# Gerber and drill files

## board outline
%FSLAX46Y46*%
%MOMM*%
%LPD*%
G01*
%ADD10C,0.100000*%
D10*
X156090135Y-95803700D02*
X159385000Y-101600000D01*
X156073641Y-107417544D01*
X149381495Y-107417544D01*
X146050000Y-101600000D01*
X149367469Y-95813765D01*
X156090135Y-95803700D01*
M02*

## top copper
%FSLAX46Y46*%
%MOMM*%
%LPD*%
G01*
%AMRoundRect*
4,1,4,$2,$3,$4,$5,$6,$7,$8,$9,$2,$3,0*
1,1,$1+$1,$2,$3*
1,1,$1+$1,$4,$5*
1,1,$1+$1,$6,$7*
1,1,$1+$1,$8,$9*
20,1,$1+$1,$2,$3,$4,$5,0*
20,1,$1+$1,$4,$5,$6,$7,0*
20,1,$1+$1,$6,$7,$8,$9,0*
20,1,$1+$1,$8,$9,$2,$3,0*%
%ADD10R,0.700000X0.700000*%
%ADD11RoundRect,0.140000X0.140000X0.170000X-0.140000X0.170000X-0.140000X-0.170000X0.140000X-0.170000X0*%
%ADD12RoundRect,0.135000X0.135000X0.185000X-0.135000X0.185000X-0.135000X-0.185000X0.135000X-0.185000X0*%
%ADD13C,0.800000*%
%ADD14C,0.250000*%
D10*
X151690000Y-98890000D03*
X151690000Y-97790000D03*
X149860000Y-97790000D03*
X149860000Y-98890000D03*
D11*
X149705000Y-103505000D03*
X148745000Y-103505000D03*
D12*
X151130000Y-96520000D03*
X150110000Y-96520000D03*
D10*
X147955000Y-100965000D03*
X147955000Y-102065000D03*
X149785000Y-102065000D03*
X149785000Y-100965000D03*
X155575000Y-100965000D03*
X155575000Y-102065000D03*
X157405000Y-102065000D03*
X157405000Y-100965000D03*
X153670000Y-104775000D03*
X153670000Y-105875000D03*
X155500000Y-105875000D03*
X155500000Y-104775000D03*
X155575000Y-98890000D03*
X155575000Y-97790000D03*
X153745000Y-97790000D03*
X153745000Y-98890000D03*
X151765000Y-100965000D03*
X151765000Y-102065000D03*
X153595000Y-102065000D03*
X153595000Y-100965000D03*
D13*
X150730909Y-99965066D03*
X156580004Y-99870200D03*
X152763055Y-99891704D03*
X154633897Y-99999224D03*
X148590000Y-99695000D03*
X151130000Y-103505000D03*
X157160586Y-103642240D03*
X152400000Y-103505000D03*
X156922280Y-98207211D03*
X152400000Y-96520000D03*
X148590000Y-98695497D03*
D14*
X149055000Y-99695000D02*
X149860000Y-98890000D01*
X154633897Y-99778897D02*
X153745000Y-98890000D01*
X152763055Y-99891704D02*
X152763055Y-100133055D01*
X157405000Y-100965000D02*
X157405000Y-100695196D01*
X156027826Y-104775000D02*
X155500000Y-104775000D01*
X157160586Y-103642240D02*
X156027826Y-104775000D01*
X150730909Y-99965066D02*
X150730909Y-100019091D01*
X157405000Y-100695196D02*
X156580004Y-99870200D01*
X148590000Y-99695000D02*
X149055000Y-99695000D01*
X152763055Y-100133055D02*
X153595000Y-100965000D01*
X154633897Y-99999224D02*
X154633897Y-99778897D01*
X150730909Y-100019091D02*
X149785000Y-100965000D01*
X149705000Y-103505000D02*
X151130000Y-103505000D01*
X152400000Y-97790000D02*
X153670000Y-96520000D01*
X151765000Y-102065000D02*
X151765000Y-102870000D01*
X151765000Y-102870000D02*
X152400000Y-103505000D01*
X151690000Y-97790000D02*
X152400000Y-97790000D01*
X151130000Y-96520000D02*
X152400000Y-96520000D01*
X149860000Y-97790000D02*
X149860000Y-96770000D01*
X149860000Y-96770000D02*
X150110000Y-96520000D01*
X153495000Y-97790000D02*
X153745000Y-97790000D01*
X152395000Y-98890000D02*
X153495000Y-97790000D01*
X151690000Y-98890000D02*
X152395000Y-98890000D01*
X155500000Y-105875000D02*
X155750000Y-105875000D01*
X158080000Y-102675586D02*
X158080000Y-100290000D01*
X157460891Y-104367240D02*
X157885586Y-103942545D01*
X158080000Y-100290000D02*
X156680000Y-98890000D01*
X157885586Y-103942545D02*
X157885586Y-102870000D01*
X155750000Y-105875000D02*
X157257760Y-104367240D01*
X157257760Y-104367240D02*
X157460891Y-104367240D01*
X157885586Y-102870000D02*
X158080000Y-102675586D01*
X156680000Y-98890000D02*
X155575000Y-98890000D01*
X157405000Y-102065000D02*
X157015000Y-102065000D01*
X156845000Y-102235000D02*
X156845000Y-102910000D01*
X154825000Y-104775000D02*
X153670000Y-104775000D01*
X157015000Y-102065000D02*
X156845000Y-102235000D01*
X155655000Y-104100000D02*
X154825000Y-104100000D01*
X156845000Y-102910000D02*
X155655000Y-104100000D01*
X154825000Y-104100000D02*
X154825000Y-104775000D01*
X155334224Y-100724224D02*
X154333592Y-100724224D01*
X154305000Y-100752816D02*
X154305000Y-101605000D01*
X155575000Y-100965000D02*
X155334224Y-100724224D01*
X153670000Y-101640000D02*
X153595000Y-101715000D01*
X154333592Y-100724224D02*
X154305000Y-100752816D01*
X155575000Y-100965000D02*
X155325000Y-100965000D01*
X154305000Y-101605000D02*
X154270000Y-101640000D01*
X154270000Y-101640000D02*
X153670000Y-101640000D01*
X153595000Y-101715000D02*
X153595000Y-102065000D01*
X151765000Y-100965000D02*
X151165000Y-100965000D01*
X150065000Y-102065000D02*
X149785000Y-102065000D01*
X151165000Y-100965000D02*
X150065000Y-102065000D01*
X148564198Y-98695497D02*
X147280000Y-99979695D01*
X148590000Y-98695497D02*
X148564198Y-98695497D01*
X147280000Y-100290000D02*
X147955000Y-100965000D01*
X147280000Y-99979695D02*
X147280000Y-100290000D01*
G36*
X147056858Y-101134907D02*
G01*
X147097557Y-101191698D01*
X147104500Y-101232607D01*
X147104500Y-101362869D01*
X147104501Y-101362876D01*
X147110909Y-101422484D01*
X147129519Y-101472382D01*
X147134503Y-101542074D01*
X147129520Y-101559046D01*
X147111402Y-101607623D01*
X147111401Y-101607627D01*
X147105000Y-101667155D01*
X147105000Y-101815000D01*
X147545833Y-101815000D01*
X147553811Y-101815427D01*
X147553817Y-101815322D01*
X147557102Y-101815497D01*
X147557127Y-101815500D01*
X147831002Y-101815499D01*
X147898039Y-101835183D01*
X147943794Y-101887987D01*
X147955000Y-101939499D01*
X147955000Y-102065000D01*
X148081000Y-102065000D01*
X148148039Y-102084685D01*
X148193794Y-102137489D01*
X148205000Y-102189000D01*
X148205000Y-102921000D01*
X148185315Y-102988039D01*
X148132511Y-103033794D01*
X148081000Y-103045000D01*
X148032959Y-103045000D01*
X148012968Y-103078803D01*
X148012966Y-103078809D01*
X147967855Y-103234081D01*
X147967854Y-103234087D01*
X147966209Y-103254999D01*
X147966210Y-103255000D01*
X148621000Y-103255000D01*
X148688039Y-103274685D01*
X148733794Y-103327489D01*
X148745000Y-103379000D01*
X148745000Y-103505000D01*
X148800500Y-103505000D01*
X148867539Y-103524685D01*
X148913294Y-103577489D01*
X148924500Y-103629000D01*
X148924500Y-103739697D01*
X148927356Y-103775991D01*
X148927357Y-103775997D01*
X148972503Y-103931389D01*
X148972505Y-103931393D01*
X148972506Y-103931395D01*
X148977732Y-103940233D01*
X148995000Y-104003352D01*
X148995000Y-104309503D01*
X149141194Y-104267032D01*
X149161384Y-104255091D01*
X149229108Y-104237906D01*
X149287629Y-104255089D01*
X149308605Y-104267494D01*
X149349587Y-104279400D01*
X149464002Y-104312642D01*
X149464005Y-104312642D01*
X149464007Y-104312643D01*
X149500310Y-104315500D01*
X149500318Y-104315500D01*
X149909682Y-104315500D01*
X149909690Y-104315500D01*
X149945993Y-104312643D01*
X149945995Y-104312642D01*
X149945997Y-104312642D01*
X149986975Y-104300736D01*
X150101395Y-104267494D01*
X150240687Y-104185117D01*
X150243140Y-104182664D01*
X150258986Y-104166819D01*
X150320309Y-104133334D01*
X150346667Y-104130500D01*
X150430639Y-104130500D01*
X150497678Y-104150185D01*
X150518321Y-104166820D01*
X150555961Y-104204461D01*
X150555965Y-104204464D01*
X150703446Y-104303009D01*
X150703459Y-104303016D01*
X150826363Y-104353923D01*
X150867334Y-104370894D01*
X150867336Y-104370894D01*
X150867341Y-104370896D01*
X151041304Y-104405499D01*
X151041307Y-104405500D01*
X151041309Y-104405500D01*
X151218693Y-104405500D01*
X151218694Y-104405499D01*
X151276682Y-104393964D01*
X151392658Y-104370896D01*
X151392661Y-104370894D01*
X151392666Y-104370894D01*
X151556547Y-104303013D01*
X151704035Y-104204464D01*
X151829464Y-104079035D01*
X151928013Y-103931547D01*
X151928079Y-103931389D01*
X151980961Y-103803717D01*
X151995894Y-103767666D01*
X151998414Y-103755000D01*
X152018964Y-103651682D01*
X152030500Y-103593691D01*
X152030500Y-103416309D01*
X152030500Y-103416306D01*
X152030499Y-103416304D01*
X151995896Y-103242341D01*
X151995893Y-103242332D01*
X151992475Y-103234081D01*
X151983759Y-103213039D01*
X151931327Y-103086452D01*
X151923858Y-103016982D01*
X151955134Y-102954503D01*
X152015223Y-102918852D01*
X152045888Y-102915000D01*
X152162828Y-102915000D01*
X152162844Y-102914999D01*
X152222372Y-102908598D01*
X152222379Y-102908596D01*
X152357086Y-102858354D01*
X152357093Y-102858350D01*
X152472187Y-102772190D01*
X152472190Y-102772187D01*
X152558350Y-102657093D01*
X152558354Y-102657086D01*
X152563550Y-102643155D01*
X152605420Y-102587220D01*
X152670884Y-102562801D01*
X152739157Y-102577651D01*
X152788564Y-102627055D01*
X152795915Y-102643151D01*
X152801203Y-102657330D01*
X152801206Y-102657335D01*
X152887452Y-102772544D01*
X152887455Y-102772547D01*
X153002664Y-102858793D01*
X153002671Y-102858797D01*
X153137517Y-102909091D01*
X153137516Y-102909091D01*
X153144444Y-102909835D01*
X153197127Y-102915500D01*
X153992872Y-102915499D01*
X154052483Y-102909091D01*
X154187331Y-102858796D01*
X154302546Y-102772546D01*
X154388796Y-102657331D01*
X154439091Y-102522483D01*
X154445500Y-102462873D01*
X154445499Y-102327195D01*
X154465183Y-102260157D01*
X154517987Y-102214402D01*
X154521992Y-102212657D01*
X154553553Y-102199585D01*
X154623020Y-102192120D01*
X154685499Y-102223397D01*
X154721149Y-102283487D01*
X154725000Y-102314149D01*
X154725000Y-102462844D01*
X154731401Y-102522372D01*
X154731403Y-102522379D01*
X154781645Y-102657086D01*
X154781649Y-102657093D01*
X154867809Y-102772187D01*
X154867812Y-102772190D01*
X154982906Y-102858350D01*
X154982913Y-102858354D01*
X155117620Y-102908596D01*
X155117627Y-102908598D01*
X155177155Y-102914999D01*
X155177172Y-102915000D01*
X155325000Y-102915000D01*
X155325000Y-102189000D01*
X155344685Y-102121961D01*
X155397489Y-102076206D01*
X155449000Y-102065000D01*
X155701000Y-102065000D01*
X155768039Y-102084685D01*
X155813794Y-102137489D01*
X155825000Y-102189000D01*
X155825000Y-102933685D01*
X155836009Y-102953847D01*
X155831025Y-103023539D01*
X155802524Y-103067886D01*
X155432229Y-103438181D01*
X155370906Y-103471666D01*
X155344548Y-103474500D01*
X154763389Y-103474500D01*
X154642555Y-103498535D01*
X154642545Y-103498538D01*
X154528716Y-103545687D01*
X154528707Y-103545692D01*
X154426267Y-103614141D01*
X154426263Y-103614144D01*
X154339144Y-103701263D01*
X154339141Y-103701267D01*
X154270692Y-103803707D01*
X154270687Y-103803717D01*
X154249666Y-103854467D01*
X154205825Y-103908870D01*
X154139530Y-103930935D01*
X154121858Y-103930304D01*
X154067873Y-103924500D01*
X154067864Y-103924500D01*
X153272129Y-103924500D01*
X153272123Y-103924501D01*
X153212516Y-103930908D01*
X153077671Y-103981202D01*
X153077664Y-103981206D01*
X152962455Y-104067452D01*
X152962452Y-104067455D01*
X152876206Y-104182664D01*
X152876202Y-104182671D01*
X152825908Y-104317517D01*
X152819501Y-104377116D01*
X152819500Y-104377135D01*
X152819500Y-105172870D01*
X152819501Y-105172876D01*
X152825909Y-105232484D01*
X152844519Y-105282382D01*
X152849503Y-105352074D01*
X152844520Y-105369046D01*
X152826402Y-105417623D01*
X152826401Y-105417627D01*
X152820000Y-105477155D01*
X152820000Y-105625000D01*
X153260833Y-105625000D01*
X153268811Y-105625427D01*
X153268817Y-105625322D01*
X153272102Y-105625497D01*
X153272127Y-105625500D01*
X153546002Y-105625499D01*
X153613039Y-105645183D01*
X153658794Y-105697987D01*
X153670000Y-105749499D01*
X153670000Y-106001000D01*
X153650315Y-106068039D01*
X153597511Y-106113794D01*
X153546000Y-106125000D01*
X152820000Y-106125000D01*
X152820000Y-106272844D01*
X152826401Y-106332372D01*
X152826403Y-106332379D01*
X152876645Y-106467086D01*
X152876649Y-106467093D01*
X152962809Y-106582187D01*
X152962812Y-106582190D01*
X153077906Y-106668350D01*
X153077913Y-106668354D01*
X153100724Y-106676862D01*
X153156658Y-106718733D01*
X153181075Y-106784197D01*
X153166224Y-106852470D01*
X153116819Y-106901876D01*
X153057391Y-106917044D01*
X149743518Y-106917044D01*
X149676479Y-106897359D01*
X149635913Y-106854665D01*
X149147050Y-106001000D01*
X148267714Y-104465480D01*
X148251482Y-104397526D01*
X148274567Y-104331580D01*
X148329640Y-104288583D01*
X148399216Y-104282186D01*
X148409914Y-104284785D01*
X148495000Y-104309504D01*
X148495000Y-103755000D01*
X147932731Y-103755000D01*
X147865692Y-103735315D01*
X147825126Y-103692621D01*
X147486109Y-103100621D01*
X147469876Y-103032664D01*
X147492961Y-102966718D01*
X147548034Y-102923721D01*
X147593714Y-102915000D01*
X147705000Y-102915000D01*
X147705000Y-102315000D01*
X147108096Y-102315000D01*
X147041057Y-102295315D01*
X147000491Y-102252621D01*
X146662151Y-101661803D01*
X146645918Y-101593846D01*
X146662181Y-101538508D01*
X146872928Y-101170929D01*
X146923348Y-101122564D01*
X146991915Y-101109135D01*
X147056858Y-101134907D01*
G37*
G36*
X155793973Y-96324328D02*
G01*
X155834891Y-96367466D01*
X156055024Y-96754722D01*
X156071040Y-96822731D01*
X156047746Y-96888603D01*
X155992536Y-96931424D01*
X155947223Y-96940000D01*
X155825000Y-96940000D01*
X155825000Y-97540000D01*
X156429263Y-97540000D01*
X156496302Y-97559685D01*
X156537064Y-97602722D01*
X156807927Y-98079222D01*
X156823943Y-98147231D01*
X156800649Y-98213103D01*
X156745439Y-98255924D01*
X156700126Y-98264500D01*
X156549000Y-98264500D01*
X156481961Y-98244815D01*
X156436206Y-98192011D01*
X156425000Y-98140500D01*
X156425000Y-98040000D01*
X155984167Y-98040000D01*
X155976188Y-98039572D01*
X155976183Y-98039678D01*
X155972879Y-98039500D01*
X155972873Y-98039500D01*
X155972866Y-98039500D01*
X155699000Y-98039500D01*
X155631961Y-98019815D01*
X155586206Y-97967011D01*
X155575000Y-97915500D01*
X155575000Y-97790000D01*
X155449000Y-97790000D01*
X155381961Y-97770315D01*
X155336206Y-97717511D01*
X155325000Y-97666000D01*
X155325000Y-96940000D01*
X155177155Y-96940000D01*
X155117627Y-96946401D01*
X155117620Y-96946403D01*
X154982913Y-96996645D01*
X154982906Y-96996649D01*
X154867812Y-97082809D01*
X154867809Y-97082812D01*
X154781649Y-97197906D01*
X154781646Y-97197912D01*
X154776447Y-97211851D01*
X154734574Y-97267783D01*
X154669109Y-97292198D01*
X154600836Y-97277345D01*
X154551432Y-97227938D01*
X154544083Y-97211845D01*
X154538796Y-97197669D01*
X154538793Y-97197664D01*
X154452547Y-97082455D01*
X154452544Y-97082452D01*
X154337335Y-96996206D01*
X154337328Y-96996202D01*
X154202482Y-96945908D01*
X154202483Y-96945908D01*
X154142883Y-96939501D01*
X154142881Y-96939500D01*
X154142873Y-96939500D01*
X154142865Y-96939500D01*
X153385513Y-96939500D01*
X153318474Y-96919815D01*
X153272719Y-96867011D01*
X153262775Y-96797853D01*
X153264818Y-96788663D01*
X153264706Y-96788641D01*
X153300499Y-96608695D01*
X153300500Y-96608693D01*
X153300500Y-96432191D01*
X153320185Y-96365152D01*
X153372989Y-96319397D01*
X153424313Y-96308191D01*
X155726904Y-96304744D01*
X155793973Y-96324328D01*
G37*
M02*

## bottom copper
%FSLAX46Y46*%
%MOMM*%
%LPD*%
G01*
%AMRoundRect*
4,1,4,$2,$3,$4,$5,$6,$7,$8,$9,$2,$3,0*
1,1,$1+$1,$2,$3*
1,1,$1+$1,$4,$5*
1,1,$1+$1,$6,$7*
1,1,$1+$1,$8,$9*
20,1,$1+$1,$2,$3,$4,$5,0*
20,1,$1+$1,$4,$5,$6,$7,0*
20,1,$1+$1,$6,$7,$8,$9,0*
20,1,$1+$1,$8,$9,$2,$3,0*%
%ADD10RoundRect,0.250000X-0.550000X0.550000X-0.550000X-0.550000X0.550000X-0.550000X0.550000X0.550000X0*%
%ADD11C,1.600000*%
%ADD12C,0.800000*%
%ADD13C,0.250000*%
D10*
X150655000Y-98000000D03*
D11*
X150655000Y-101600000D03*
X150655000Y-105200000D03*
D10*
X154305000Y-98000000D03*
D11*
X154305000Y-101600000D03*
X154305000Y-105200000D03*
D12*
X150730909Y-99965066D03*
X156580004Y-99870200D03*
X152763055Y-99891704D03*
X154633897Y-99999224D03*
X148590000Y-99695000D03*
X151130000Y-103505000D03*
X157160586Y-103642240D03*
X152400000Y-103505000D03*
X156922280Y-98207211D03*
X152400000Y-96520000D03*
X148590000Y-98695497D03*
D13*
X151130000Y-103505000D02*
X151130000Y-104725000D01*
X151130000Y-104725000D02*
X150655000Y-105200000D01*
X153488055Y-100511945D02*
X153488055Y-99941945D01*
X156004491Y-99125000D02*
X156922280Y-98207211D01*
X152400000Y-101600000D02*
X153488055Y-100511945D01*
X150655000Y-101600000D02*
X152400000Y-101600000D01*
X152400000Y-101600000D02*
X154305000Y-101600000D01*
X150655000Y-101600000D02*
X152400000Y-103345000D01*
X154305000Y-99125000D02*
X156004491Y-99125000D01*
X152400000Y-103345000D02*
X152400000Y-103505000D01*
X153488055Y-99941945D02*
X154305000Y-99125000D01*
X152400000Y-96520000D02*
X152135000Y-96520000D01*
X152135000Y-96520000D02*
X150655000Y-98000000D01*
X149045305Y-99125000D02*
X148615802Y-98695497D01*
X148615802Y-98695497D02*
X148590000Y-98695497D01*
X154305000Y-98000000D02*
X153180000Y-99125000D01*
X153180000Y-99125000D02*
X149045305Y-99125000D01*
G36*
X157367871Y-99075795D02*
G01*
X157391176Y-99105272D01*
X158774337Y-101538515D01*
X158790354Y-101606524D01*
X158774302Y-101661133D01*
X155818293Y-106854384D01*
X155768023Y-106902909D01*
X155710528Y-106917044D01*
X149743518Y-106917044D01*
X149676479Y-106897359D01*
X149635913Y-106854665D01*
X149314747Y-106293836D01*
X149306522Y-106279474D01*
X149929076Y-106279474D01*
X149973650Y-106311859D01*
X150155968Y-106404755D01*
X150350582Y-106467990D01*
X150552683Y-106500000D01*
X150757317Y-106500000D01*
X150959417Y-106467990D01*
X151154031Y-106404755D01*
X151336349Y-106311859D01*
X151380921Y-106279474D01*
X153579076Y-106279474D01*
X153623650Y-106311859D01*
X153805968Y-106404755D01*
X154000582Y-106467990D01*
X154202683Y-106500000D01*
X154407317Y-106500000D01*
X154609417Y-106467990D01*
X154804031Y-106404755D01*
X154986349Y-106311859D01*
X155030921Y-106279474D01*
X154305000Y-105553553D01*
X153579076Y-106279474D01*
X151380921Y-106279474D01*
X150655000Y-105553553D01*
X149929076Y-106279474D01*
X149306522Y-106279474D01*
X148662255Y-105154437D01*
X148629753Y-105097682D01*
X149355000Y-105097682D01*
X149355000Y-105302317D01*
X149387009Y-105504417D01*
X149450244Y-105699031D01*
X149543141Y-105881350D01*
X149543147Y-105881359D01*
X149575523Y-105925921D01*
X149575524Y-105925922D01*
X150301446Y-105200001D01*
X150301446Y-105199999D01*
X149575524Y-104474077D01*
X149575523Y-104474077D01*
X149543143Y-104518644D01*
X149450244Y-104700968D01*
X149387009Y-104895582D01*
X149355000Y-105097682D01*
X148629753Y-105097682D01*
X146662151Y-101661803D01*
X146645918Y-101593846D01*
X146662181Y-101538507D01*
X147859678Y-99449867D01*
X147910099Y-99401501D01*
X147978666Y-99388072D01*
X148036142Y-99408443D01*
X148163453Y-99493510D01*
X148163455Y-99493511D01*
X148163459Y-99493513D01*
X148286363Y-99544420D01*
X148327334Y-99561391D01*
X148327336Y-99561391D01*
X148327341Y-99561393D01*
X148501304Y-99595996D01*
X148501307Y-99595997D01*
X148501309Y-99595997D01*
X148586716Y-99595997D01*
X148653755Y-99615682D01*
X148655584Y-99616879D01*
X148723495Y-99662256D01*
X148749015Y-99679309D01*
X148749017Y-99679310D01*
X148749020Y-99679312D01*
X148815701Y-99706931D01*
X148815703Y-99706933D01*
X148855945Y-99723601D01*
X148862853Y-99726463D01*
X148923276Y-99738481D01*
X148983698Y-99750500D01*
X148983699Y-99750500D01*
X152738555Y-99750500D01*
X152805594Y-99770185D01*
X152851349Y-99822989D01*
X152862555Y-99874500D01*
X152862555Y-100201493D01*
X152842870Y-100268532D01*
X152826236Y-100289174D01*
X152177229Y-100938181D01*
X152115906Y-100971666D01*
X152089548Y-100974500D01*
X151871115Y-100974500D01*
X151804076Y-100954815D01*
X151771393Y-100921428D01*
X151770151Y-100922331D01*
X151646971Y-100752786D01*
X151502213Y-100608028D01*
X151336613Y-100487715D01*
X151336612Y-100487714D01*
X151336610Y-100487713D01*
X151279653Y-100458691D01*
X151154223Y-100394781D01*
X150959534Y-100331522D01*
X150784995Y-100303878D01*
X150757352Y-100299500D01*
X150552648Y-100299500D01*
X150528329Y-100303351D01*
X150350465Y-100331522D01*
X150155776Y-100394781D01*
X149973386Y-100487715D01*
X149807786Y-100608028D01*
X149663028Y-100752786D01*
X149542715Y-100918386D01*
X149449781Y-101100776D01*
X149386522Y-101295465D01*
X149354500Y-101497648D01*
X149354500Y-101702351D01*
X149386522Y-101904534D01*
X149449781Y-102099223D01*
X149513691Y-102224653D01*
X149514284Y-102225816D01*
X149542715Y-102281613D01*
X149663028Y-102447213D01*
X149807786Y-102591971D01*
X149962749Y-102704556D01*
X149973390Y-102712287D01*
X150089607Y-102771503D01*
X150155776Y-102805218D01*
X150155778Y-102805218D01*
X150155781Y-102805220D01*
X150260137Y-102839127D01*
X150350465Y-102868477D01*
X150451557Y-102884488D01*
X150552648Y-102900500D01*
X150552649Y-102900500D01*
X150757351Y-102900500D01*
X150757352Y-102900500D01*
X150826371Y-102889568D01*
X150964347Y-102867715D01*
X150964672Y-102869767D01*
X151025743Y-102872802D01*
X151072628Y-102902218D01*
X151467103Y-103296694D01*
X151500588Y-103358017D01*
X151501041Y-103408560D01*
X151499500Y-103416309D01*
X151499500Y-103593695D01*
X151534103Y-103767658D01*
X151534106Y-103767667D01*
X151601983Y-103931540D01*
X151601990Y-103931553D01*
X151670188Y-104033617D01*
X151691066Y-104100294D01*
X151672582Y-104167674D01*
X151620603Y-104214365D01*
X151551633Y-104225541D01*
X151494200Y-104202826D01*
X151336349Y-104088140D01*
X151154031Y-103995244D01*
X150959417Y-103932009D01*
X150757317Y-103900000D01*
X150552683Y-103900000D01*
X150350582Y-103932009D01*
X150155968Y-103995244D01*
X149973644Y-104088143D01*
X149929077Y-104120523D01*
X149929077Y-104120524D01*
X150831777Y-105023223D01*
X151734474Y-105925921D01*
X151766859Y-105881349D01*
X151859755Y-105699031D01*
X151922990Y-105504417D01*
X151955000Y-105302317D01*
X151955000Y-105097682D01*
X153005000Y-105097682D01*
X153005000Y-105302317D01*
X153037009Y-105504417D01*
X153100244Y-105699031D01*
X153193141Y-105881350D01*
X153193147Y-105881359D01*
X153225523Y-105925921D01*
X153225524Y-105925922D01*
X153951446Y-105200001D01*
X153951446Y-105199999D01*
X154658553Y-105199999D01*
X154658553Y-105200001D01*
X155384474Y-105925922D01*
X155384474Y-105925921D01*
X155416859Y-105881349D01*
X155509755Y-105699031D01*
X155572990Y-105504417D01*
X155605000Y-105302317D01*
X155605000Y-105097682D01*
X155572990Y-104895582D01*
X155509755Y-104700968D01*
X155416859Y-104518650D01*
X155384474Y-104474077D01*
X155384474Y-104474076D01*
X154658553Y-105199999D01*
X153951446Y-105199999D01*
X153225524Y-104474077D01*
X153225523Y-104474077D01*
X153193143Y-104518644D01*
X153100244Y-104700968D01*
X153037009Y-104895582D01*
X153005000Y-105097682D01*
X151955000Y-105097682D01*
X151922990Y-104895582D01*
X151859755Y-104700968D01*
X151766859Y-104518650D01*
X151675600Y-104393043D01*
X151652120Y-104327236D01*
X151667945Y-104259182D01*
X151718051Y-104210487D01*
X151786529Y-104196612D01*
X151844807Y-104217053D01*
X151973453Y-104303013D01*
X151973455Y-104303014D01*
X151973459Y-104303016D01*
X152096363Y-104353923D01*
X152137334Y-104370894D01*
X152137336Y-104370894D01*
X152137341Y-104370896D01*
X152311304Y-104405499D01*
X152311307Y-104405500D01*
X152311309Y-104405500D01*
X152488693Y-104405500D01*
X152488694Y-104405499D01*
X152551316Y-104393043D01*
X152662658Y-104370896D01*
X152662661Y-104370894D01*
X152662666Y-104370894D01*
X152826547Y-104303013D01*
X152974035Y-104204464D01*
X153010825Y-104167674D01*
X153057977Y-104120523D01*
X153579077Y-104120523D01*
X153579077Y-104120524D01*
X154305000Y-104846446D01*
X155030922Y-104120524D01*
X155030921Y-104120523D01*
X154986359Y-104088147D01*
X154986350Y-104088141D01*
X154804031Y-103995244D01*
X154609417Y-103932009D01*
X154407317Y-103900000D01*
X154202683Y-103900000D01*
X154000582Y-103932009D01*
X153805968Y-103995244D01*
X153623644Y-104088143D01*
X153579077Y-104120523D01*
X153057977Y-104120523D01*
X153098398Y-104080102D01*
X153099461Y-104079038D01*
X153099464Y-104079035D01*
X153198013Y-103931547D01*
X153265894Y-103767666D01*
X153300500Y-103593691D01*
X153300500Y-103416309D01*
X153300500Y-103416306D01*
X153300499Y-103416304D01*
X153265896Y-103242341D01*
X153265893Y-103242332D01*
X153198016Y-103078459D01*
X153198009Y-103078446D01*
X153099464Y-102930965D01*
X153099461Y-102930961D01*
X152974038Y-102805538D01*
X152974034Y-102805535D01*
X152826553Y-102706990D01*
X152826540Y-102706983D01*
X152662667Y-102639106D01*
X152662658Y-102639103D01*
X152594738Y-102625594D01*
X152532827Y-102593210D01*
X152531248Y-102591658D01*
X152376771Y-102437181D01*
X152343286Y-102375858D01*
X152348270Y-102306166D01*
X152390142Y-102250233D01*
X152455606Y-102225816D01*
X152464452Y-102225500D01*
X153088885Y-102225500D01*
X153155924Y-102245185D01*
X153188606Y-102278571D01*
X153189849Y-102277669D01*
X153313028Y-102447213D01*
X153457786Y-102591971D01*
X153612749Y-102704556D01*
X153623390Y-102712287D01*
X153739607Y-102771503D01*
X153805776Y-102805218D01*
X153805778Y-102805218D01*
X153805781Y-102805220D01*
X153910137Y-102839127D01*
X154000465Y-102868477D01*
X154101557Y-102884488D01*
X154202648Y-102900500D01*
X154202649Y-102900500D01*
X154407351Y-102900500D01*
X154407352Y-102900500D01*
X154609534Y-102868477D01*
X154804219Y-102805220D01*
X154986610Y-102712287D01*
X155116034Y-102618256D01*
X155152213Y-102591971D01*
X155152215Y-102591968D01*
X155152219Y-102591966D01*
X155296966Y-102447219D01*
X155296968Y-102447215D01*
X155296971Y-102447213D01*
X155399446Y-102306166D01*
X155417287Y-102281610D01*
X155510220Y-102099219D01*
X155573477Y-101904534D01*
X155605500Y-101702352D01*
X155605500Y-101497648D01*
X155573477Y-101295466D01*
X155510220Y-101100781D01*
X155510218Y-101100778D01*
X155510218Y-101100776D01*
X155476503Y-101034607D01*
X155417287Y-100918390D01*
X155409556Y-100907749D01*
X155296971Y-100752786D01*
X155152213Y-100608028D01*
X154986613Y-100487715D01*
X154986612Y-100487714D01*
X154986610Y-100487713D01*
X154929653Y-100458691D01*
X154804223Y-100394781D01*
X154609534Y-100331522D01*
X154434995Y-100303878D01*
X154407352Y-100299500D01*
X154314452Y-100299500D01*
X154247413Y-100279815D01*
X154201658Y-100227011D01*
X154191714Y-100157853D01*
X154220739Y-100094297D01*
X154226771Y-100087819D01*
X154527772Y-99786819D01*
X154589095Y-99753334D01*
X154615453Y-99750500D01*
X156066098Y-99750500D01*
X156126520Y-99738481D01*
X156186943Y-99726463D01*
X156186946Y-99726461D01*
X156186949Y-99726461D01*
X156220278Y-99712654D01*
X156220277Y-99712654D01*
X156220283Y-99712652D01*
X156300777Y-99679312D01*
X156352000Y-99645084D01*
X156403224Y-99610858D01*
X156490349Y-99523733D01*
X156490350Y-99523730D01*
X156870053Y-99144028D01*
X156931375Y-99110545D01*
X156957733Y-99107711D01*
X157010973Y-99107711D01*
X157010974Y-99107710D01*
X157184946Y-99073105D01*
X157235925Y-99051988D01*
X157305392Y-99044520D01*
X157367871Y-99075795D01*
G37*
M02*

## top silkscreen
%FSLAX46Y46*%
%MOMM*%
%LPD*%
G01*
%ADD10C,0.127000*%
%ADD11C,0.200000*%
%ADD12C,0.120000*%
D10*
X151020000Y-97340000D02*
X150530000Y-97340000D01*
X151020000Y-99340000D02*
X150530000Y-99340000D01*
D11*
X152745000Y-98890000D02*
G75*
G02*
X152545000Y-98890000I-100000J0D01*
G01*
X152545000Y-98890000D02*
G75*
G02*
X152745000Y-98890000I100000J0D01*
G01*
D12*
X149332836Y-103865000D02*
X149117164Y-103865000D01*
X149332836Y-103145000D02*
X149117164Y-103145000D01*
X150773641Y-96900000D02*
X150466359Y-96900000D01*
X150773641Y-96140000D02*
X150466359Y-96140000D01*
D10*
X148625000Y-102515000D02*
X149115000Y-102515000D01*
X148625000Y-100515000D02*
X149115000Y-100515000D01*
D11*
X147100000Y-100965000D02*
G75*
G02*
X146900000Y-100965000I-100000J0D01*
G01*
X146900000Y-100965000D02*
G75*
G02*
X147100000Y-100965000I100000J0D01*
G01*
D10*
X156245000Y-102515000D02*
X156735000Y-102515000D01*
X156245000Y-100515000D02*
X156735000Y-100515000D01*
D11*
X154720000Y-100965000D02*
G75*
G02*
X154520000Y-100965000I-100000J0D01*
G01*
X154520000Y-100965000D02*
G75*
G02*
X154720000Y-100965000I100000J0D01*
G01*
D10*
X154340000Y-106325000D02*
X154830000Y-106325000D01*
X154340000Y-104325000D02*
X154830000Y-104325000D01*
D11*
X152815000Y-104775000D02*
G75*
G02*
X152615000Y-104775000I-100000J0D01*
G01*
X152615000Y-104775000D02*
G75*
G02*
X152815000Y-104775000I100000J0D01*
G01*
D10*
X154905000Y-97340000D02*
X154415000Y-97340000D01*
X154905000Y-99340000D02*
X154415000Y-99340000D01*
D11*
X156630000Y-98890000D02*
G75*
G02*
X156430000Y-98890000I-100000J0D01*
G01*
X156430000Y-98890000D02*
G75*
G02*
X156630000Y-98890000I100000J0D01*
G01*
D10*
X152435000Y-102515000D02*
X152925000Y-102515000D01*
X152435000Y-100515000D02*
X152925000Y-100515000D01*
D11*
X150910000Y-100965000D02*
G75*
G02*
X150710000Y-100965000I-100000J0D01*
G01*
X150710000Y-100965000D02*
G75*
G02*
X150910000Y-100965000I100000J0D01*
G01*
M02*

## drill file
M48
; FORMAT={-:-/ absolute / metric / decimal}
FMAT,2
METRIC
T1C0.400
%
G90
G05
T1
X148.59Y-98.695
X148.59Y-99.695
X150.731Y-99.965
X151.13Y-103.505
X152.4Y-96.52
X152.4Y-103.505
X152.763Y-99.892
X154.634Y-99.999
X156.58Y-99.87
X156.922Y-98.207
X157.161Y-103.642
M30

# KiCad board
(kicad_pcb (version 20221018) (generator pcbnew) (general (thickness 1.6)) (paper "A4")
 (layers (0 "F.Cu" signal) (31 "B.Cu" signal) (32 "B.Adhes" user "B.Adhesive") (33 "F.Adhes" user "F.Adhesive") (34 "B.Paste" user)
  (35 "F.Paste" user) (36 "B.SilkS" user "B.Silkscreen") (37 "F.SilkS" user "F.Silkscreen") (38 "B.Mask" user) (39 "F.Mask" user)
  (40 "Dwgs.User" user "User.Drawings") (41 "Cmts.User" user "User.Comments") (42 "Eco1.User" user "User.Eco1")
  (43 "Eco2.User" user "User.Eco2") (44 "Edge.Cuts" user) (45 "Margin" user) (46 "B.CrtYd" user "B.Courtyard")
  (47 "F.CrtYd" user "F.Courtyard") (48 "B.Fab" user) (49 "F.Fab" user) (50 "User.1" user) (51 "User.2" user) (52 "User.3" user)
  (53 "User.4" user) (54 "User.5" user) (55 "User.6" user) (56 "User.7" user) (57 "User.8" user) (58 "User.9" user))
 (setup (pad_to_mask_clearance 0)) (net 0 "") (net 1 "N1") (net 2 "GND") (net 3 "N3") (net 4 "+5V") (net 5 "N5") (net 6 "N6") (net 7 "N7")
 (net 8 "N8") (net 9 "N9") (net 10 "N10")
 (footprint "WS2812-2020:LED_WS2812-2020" (layer "F.Cu") (at 150.775 98.34)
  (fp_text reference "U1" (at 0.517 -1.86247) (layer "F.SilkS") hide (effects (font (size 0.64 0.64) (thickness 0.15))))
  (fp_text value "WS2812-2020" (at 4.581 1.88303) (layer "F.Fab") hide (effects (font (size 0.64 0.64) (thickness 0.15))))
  (fp_line (start 0.245 -1) (end -0.245 -1) (stroke (width 0.127) (type solid)) (layer "F.SilkS"))
  (fp_line (start 0.245 1) (end -0.245 1) (stroke (width 0.127) (type solid)) (layer "F.SilkS"))
  (fp_circle (center 1.87 0.55) (end 1.97 0.55) (stroke (width 0.2) (type solid)) (fill none) (layer "F.SilkS"))
  (pad "1" smd rect (at 0.915 0.55) (size 0.7 0.7) (layers "F.Cu" "F.Paste" "F.Mask") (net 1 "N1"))
  (pad "2" smd rect (at 0.915 -0.55) (size 0.7 0.7) (layers "F.Cu" "F.Paste" "F.Mask") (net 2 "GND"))
  (pad "3" smd rect (at -0.915 -0.55) (size 0.7 0.7) (layers "F.Cu" "F.Paste" "F.Mask") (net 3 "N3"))
  (pad "4" smd rect (at -0.915 0.55) (size 0.7 0.7) (layers "F.Cu" "F.Paste" "F.Mask") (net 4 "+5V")))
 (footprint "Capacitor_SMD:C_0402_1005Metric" (layer "F.Cu") (at 149.225 103.505 180)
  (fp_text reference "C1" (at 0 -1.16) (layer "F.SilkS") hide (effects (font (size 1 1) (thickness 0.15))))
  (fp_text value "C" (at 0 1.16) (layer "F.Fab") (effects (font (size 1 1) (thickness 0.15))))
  (fp_line (start -0.107836 -0.36) (end 0.107836 -0.36) (stroke (width 0.12) (type solid)) (layer "F.SilkS"))
  (fp_line (start -0.107836 0.36) (end 0.107836 0.36) (stroke (width 0.12) (type solid)) (layer "F.SilkS"))
  (pad "1" smd roundrect (at -0.48 0 180) (size 0.56 0.62) (layers "F.Cu" "F.Paste" "F.Mask") (roundrect_rratio 0.25) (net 4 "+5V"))
  (pad "2" smd roundrect (at 0.48 0 180) (size 0.56 0.62) (layers "F.Cu" "F.Paste" "F.Mask") (roundrect_rratio 0.25) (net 2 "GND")))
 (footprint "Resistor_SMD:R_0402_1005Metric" (layer "F.Cu") (at 150.62 96.52 180)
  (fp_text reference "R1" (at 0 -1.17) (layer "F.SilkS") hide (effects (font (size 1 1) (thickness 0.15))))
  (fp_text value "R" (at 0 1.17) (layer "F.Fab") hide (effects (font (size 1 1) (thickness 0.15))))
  (fp_line (start -0.153641 -0.38) (end 0.153641 -0.38) (stroke (width 0.12) (type solid)) (layer "F.SilkS"))
  (fp_line (start -0.153641 0.38) (end 0.153641 0.38) (stroke (width 0.12) (type solid)) (layer "F.SilkS"))
  (pad "1" smd roundrect (at -0.51 0 180) (size 0.54 0.64) (layers "F.Cu" "F.Paste" "F.Mask") (roundrect_rratio 0.25) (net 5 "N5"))
  (pad "2" smd roundrect (at 0.51 0 180) (size 0.54 0.64) (layers "F.Cu" "F.Paste" "F.Mask") (roundrect_rratio 0.25) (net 3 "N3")))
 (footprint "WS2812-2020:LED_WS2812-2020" (layer "F.Cu") (at 148.87 101.515 180)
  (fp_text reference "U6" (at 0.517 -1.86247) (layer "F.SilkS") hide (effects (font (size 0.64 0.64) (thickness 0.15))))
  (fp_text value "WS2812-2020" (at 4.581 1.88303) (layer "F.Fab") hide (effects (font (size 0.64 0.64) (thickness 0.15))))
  (fp_line (start 0.245 -1) (end -0.245 -1) (stroke (width 0.127) (type solid)) (layer "F.SilkS"))
  (fp_line (start 0.245 1) (end -0.245 1) (stroke (width 0.127) (type solid)) (layer "F.SilkS"))
  (fp_circle (center 1.87 0.55) (end 1.97 0.55) (stroke (width 0.2) (type solid)) (fill none) (layer "F.SilkS"))
  (pad "1" smd rect (at 0.915 0.55 180) (size 0.7 0.7) (layers "F.Cu" "F.Paste" "F.Mask") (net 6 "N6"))
  (pad "2" smd rect (at 0.915 -0.55 180) (size 0.7 0.7) (layers "F.Cu" "F.Paste" "F.Mask") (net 2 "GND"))
  (pad "3" smd rect (at -0.915 -0.55 180) (size 0.7 0.7) (layers "F.Cu" "F.Paste" "F.Mask") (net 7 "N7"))
  (pad "4" smd rect (at -0.915 0.55 180) (size 0.7 0.7) (layers "F.Cu" "F.Paste" "F.Mask") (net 4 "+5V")))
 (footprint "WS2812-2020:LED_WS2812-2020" (layer "F.Cu") (at 156.49 101.515 180)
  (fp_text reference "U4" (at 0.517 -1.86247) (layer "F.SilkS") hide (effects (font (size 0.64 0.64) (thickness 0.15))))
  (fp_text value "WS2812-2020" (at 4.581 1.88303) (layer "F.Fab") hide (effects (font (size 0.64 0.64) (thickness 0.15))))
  (fp_line (start 0.245 -1) (end -0.245 -1) (stroke (width 0.127) (type solid)) (layer "F.SilkS"))
  (fp_line (start 0.245 1) (end -0.245 1) (stroke (width 0.127) (type solid)) (layer "F.SilkS"))
  (fp_circle (center 1.87 0.55) (end 1.97 0.55) (stroke (width 0.2) (type solid)) (fill none) (layer "F.SilkS"))
  (pad "1" smd rect (at 0.915 0.55 180) (size 0.7 0.7) (layers "F.Cu" "F.Paste" "F.Mask") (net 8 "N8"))
  (pad "2" smd rect (at 0.915 -0.55 180) (size 0.7 0.7) (layers "F.Cu" "F.Paste" "F.Mask") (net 2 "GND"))
  (pad "3" smd rect (at -0.915 -0.55 180) (size 0.7 0.7) (layers "F.Cu" "F.Paste" "F.Mask") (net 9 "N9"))
  (pad "4" smd rect (at -0.915 0.55 180) (size 0.7 0.7) (layers "F.Cu" "F.Paste" "F.Mask") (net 4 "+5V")))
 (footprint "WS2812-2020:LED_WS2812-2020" (layer "F.Cu") (at 154.585 105.325 180)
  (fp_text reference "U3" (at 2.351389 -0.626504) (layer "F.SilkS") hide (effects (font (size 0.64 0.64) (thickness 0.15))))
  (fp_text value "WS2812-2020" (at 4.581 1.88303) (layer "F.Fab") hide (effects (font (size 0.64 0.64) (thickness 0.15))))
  (fp_line (start 0.245 -1) (end -0.245 -1) (stroke (width 0.127) (type solid)) (layer "F.SilkS"))
  (fp_line (start 0.245 1) (end -0.245 1) (stroke (width 0.127) (type solid)) (layer "F.SilkS"))
  (fp_circle (center 1.87 0.55) (end 1.97 0.55) (stroke (width 0.2) (type solid)) (fill none) (layer "F.SilkS"))
  (pad "1" smd rect (at 0.915 0.55 180) (size 0.7 0.7) (layers "F.Cu" "F.Paste" "F.Mask") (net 9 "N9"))
  (pad "2" smd rect (at 0.915 -0.55 180) (size 0.7 0.7) (layers "F.Cu" "F.Paste" "F.Mask") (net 2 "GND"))
  (pad "3" smd rect (at -0.915 -0.55 180) (size 0.7 0.7) (layers "F.Cu" "F.Paste" "F.Mask") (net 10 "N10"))
  (pad "4" smd rect (at -0.915 0.55 180) (size 0.7 0.7) (layers "F.Cu" "F.Paste" "F.Mask") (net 4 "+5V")))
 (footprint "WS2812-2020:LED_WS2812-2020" (layer "F.Cu") (at 154.66 98.34)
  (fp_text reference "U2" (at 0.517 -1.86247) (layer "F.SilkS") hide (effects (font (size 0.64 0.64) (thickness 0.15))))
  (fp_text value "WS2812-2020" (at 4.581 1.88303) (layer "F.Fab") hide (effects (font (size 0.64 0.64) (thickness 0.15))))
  (fp_line (start 0.245 -1) (end -0.245 -1) (stroke (width 0.127) (type solid)) (layer "F.SilkS"))
  (fp_line (start 0.245 1) (end -0.245 1) (stroke (width 0.127) (type solid)) (layer "F.SilkS"))
  (fp_circle (center 1.87 0.55) (end 1.97 0.55) (stroke (width 0.2) (type solid)) (fill none) (layer "F.SilkS"))
  (pad "1" smd rect (at 0.915 0.55) (size 0.7 0.7) (layers "F.Cu" "F.Paste" "F.Mask") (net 10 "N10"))
  (pad "2" smd rect (at 0.915 -0.55) (size 0.7 0.7) (layers "F.Cu" "F.Paste" "F.Mask") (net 2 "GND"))
  (pad "3" smd rect (at -0.915 -0.55) (size 0.7 0.7) (layers "F.Cu" "F.Paste" "F.Mask") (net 1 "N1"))
  (pad "4" smd rect (at -0.915 0.55) (size 0.7 0.7) (layers "F.Cu" "F.Paste" "F.Mask") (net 4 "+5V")))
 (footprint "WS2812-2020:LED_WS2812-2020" (layer "F.Cu") (at 152.68 101.515 180)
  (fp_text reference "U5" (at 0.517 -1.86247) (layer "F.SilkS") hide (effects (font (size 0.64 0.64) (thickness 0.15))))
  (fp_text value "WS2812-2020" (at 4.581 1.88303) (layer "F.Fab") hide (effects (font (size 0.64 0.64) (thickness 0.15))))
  (fp_line (start 0.245 -1) (end -0.245 -1) (stroke (width 0.127) (type solid)) (layer "F.SilkS"))
  (fp_line (start 0.245 1) (end -0.245 1) (stroke (width 0.127) (type solid)) (layer "F.SilkS"))
  (fp_circle (center 1.87 0.55) (end 1.97 0.55) (stroke (width 0.2) (type solid)) (fill none) (layer "F.SilkS"))
  (pad "1" smd rect (at 0.915 0.55 180) (size 0.7 0.7) (layers "F.Cu" "F.Paste" "F.Mask") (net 7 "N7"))
  (pad "2" smd rect (at 0.915 -0.55 180) (size 0.7 0.7) (layers "F.Cu" "F.Paste" "F.Mask") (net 2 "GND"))
  (pad "3" smd rect (at -0.915 -0.55 180) (size 0.7 0.7) (layers "F.Cu" "F.Paste" "F.Mask") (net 8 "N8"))
  (pad "4" smd rect (at -0.915 0.55 180) (size 0.7 0.7) (layers "F.Cu" "F.Paste" "F.Mask") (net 4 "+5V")))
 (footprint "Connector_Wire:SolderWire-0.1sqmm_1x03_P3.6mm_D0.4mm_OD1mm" (layer "B.Cu") (at 150.655 98 -90)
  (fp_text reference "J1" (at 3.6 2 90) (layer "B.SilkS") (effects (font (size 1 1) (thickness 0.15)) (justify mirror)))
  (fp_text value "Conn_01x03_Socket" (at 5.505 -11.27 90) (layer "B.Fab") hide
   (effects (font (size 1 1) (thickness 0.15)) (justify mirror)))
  (pad "1" connect roundrect (at 0 0 270) (size 1.6 1.6) (layers "B.Cu" "B.Mask") (roundrect_rratio 0.15625) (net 5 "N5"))
  (pad "2" connect circle (at 3.6 0 270) (size 1.6 1.6) (layers "B.Cu" "B.Mask") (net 2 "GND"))
  (pad "3" connect circle (at 7.2 0) (size 1.6 1.6) (layers "B.Cu" "B.Mask") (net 4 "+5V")))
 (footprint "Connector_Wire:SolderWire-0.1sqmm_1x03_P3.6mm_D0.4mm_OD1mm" (layer "B.Cu") (at 154.305 98 -90)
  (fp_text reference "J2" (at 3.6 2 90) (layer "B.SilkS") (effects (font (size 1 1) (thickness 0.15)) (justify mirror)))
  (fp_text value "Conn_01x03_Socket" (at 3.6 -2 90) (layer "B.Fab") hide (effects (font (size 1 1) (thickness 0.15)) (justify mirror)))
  (pad "1" connect roundrect (at 0 0 270) (size 1.6 1.6) (layers "B.Cu" "B.Mask") (roundrect_rratio 0.15625) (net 6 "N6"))
  (pad "2" connect circle (at 3.6 0 270) (size 1.6 1.6) (layers "B.Cu" "B.Mask") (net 2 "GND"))
  (pad "3" connect circle (at 7.2 0 270) (size 1.6 1.6) (layers "B.Cu" "B.Mask") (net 4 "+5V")))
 (gr_poly
  (pts (xy 156.090135 95.8037) (xy 159.385 101.6) (xy 156.073641 107.417544) (xy 149.381495 107.417544) (xy 146.05 101.6)
   (xy 149.367469 95.813765))
  (stroke (width 0.1) (type solid)) (fill none) (layer "Edge.Cuts"))
 (segment (start 149.055 99.695) (end 149.86 98.89) (width 0.25) (layer "F.Cu") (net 4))
 (segment (start 154.633897 99.778897) (end 153.745 98.89) (width 0.25) (layer "F.Cu") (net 4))
 (segment (start 152.763055 99.891704) (end 152.763055 100.133055) (width 0.25) (layer "F.Cu") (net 4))
 (segment (start 157.405 100.965) (end 157.405 100.695196) (width 0.25) (layer "F.Cu") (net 4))
 (segment (start 156.027826 104.775) (end 155.5 104.775) (width 0.25) (layer "F.Cu") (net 4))
 (segment (start 157.160586 103.64224) (end 156.027826 104.775) (width 0.25) (layer "F.Cu") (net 4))
 (segment (start 150.730909 99.965066) (end 150.730909 100.019091) (width 0.25) (layer "F.Cu") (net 4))
 (segment (start 157.405 100.695196) (end 156.580004 99.8702) (width 0.25) (layer "F.Cu") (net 4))
 (segment (start 148.59 99.695) (end 149.055 99.695) (width 0.25) (layer "F.Cu") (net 4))
 (segment (start 152.763055 100.133055) (end 153.595 100.965) (width 0.25) (layer "F.Cu") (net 4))
 (segment (start 154.633897 99.999224) (end 154.633897 99.778897) (width 0.25) (layer "F.Cu") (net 4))
 (segment (start 150.730909 100.019091) (end 149.785 100.965) (width 0.25) (layer "F.Cu") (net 4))
 (segment (start 149.705 103.505) (end 151.13 103.505) (width 0.25) (layer "F.Cu") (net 4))
 (via (at 150.730909 99.965066) (size 0.8) (drill 0.4) (layers "F.Cu" "B.Cu") (free) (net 4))
 (via (at 156.580004 99.8702) (size 0.8) (drill 0.4) (layers "F.Cu" "B.Cu") (free) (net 4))
 (via (at 152.763055 99.891704) (size 0.8) (drill 0.4) (layers "F.Cu" "B.Cu") (free) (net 4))
 (via (at 154.633897 99.999224) (size 0.8) (drill 0.4) (layers "F.Cu" "B.Cu") (free) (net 4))
 (via (at 148.59 99.695) (size 0.8) (drill 0.4) (layers "F.Cu" "B.Cu") (free) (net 4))
 (via (at 151.13 103.505) (size 0.8) (drill 0.4) (layers "F.Cu" "B.Cu") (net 4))
 (via (at 157.160586 103.64224) (size 0.8) (drill 0.4) (layers "F.Cu" "B.Cu") (free) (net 4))
 (segment (start 151.13 103.505) (end 151.13 104.725) (width 0.25) (layer "B.Cu") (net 4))
 (segment (start 151.13 104.725) (end 150.655 105.2) (width 0.25) (layer "B.Cu") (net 4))
 (segment (start 152.4 97.79) (end 153.67 96.52) (width 0.25) (layer "F.Cu") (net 2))
 (segment (start 151.765 102.065) (end 151.765 102.87) (width 0.25) (layer "F.Cu") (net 2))
 (segment (start 151.765 102.87) (end 152.4 103.505) (width 0.25) (layer "F.Cu") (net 2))
 (segment (start 151.69 97.79) (end 152.4 97.79) (width 0.25) (layer "F.Cu") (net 2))
 (via (at 152.4 103.505) (size 0.8) (drill 0.4) (layers "F.Cu" "B.Cu") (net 2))
 (via (at 156.92228 98.207211) (size 0.8) (drill 0.4) (layers "F.Cu" "B.Cu") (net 2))
 (segment (start 153.488055 100.511945) (end 153.488055 99.941945) (width 0.25) (layer "B.Cu") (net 2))
 (segment (start 156.004491 99.125) (end 156.92228 98.207211) (width 0.25) (layer "B.Cu") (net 2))
 (segment (start 152.4 101.6) (end 153.488055 100.511945) (width 0.25) (layer "B.Cu") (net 2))
 (segment (start 150.655 101.6) (end 152.4 101.6) (width 0.25) (layer "B.Cu") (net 2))
 (segment (start 152.4 101.6) (end 154.305 101.6) (width 0.25) (layer "B.Cu") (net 2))
 (segment (start 150.655 101.6) (end 152.4 103.345) (width 0.25) (layer "B.Cu") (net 2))
 (segment (start 154.305 99.125) (end 156.004491 99.125) (width 0.25) (layer "B.Cu") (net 2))
 (segment (start 152.4 103.345) (end 152.4 103.505) (width 0.25) (layer "B.Cu") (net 2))
 (segment (start 153.488055 99.941945) (end 154.305 99.125) (width 0.25) (layer "B.Cu") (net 2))
 (segment (start 151.13 96.52) (end 152.4 96.52) (width 0.25) (layer "F.Cu") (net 5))
 (via (at 152.4 96.52) (size 0.8) (drill 0.4) (layers "F.Cu" "B.Cu") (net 5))
 (segment (start 152.4 96.52) (end 152.135 96.52) (width 0.25) (layer "B.Cu") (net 5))
 (segment (start 152.135 96.52) (end 150.655 98) (width 0.25) (layer "B.Cu") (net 5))
 (segment (start 149.86 97.79) (end 149.86 96.77) (width 0.25) (layer "F.Cu") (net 3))
 (segment (start 149.86 96.77) (end 150.11 96.52) (width 0.25) (layer "F.Cu") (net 3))
 (segment (start 153.495 97.79) (end 153.745 97.79) (width 0.25) (layer "F.Cu") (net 1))
 (segment (start 152.395 98.89) (end 153.495 97.79) (width 0.25) (layer "F.Cu") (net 1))
 (segment (start 151.69 98.89) (end 152.395 98.89) (width 0.25) (layer "F.Cu") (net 1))
 (segment (start 155.5 105.875) (end 155.75 105.875) (width 0.25) (layer "F.Cu") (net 10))
 (segment (start 158.08 102.675586) (end 158.08 100.29) (width 0.25) (layer "F.Cu") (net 10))
 (segment (start 157.460891 104.36724) (end 157.885586 103.942545) (width 0.25) (layer "F.Cu") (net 10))
 (segment (start 158.08 100.29) (end 156.68 98.89) (width 0.25) (layer "F.Cu") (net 10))
 (segment (start 157.885586 103.942545) (end 157.885586 102.87) (width 0.25) (layer "F.Cu") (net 10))
 (segment (start 155.75 105.875) (end 157.25776 104.36724) (width 0.25) (layer "F.Cu") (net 10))
 (segment (start 157.25776 104.36724) (end 157.460891 104.36724) (width 0.25) (layer "F.Cu") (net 10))
 (segment (start 157.885586 102.87) (end 158.08 102.675586) (width 0.25) (layer "F.Cu") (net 10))
 (segment (start 156.68 98.89) (end 155.575 98.89) (width 0.25) (layer "F.Cu") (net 10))
 (segment (start 157.405 102.065) (end 157.015 102.065) (width 0.25) (layer "F.Cu") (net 9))
 (segment (start 156.845 102.235) (end 156.845 102.91) (width 0.25) (layer "F.Cu") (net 9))
 (segment (start 154.825 104.775) (end 153.67 104.775) (width 0.25) (layer "F.Cu") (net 9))
 (segment (start 157.015 102.065) (end 156.845 102.235) (width 0.25) (layer "F.Cu") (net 9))
 (segment (start 155.655 104.1) (end 154.825 104.1) (width 0.25) (layer "F.Cu") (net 9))
 (segment (start 156.845 102.91) (end 155.655 104.1) (width 0.25) (layer "F.Cu") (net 9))
 (segment (start 154.825 104.1) (end 154.825 104.775) (width 0.25) (layer "F.Cu") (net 9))
 (segment (start 155.334224 100.724224) (end 154.333592 100.724224) (width 0.25) (layer "F.Cu") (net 8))
 (segment (start 154.305 100.752816) (end 154.305 101.605) (width 0.25) (layer "F.Cu") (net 8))
 (segment (start 155.575 100.965) (end 155.334224 100.724224) (width 0.25) (layer "F.Cu") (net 8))
 (segment (start 153.67 101.64) (end 153.595 101.715) (width 0.25) (layer "F.Cu") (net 8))
 (segment (start 154.333592 100.724224) (end 154.305 100.752816) (width 0.25) (layer "F.Cu") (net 8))
 (segment (start 155.575 100.965) (end 155.325 100.965) (width 0.25) (layer "F.Cu") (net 8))
 (segment (start 154.305 101.605) (end 154.27 101.64) (width 0.25) (layer "F.Cu") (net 8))
 (segment (start 154.27 101.64) (end 153.67 101.64) (width 0.25) (layer "F.Cu") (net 8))
 (segment (start 153.595 101.715) (end 153.595 102.065) (width 0.25) (layer "F.Cu") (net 8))
 (segment (start 151.765 100.965) (end 151.165 100.965) (width 0.25) (layer "F.Cu") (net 7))
 (segment (start 150.065 102.065) (end 149.785 102.065) (width 0.25) (layer "F.Cu") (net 7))
 (segment (start 151.165 100.965) (end 150.065 102.065) (width 0.25) (layer "F.Cu") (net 7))
 (segment (start 148.564198 98.695497) (end 147.28 99.979695) (width 0.25) (layer "F.Cu") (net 6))
 (segment (start 148.59 98.695497) (end 148.564198 98.695497) (width 0.25) (layer "F.Cu") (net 6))
 (segment (start 147.28 100.29) (end 147.955 100.965) (width 0.25) (layer "F.Cu") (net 6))
 (segment (start 147.28 99.979695) (end 147.28 100.29) (width 0.25) (layer "F.Cu") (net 6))
 (via (at 148.59 98.695497) (size 0.8) (drill 0.4) (layers "F.Cu" "B.Cu") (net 6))
 (segment (start 149.045305 99.125) (end 148.615802 98.695497) (width 0.25) (layer "B.Cu") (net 6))
 (segment (start 148.615802 98.695497) (end 148.59 98.695497) (width 0.25) (layer "B.Cu") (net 6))
 (segment (start 154.305 98) (end 153.18 99.125) (width 0.25) (layer "B.Cu") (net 6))
 (segment (start 153.18 99.125) (end 149.045305 99.125) (width 0.25) (layer "B.Cu") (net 6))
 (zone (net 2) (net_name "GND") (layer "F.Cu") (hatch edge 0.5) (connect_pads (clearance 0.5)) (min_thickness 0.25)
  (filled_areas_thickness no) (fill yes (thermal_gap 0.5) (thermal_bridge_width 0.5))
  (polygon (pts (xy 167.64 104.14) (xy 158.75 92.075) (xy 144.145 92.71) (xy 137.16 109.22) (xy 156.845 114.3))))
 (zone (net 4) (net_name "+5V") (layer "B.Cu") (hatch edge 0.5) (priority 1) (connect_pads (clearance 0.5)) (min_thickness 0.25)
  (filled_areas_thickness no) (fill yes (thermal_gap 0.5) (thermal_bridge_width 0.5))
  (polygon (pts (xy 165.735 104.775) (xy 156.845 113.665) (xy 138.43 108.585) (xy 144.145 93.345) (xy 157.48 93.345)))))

